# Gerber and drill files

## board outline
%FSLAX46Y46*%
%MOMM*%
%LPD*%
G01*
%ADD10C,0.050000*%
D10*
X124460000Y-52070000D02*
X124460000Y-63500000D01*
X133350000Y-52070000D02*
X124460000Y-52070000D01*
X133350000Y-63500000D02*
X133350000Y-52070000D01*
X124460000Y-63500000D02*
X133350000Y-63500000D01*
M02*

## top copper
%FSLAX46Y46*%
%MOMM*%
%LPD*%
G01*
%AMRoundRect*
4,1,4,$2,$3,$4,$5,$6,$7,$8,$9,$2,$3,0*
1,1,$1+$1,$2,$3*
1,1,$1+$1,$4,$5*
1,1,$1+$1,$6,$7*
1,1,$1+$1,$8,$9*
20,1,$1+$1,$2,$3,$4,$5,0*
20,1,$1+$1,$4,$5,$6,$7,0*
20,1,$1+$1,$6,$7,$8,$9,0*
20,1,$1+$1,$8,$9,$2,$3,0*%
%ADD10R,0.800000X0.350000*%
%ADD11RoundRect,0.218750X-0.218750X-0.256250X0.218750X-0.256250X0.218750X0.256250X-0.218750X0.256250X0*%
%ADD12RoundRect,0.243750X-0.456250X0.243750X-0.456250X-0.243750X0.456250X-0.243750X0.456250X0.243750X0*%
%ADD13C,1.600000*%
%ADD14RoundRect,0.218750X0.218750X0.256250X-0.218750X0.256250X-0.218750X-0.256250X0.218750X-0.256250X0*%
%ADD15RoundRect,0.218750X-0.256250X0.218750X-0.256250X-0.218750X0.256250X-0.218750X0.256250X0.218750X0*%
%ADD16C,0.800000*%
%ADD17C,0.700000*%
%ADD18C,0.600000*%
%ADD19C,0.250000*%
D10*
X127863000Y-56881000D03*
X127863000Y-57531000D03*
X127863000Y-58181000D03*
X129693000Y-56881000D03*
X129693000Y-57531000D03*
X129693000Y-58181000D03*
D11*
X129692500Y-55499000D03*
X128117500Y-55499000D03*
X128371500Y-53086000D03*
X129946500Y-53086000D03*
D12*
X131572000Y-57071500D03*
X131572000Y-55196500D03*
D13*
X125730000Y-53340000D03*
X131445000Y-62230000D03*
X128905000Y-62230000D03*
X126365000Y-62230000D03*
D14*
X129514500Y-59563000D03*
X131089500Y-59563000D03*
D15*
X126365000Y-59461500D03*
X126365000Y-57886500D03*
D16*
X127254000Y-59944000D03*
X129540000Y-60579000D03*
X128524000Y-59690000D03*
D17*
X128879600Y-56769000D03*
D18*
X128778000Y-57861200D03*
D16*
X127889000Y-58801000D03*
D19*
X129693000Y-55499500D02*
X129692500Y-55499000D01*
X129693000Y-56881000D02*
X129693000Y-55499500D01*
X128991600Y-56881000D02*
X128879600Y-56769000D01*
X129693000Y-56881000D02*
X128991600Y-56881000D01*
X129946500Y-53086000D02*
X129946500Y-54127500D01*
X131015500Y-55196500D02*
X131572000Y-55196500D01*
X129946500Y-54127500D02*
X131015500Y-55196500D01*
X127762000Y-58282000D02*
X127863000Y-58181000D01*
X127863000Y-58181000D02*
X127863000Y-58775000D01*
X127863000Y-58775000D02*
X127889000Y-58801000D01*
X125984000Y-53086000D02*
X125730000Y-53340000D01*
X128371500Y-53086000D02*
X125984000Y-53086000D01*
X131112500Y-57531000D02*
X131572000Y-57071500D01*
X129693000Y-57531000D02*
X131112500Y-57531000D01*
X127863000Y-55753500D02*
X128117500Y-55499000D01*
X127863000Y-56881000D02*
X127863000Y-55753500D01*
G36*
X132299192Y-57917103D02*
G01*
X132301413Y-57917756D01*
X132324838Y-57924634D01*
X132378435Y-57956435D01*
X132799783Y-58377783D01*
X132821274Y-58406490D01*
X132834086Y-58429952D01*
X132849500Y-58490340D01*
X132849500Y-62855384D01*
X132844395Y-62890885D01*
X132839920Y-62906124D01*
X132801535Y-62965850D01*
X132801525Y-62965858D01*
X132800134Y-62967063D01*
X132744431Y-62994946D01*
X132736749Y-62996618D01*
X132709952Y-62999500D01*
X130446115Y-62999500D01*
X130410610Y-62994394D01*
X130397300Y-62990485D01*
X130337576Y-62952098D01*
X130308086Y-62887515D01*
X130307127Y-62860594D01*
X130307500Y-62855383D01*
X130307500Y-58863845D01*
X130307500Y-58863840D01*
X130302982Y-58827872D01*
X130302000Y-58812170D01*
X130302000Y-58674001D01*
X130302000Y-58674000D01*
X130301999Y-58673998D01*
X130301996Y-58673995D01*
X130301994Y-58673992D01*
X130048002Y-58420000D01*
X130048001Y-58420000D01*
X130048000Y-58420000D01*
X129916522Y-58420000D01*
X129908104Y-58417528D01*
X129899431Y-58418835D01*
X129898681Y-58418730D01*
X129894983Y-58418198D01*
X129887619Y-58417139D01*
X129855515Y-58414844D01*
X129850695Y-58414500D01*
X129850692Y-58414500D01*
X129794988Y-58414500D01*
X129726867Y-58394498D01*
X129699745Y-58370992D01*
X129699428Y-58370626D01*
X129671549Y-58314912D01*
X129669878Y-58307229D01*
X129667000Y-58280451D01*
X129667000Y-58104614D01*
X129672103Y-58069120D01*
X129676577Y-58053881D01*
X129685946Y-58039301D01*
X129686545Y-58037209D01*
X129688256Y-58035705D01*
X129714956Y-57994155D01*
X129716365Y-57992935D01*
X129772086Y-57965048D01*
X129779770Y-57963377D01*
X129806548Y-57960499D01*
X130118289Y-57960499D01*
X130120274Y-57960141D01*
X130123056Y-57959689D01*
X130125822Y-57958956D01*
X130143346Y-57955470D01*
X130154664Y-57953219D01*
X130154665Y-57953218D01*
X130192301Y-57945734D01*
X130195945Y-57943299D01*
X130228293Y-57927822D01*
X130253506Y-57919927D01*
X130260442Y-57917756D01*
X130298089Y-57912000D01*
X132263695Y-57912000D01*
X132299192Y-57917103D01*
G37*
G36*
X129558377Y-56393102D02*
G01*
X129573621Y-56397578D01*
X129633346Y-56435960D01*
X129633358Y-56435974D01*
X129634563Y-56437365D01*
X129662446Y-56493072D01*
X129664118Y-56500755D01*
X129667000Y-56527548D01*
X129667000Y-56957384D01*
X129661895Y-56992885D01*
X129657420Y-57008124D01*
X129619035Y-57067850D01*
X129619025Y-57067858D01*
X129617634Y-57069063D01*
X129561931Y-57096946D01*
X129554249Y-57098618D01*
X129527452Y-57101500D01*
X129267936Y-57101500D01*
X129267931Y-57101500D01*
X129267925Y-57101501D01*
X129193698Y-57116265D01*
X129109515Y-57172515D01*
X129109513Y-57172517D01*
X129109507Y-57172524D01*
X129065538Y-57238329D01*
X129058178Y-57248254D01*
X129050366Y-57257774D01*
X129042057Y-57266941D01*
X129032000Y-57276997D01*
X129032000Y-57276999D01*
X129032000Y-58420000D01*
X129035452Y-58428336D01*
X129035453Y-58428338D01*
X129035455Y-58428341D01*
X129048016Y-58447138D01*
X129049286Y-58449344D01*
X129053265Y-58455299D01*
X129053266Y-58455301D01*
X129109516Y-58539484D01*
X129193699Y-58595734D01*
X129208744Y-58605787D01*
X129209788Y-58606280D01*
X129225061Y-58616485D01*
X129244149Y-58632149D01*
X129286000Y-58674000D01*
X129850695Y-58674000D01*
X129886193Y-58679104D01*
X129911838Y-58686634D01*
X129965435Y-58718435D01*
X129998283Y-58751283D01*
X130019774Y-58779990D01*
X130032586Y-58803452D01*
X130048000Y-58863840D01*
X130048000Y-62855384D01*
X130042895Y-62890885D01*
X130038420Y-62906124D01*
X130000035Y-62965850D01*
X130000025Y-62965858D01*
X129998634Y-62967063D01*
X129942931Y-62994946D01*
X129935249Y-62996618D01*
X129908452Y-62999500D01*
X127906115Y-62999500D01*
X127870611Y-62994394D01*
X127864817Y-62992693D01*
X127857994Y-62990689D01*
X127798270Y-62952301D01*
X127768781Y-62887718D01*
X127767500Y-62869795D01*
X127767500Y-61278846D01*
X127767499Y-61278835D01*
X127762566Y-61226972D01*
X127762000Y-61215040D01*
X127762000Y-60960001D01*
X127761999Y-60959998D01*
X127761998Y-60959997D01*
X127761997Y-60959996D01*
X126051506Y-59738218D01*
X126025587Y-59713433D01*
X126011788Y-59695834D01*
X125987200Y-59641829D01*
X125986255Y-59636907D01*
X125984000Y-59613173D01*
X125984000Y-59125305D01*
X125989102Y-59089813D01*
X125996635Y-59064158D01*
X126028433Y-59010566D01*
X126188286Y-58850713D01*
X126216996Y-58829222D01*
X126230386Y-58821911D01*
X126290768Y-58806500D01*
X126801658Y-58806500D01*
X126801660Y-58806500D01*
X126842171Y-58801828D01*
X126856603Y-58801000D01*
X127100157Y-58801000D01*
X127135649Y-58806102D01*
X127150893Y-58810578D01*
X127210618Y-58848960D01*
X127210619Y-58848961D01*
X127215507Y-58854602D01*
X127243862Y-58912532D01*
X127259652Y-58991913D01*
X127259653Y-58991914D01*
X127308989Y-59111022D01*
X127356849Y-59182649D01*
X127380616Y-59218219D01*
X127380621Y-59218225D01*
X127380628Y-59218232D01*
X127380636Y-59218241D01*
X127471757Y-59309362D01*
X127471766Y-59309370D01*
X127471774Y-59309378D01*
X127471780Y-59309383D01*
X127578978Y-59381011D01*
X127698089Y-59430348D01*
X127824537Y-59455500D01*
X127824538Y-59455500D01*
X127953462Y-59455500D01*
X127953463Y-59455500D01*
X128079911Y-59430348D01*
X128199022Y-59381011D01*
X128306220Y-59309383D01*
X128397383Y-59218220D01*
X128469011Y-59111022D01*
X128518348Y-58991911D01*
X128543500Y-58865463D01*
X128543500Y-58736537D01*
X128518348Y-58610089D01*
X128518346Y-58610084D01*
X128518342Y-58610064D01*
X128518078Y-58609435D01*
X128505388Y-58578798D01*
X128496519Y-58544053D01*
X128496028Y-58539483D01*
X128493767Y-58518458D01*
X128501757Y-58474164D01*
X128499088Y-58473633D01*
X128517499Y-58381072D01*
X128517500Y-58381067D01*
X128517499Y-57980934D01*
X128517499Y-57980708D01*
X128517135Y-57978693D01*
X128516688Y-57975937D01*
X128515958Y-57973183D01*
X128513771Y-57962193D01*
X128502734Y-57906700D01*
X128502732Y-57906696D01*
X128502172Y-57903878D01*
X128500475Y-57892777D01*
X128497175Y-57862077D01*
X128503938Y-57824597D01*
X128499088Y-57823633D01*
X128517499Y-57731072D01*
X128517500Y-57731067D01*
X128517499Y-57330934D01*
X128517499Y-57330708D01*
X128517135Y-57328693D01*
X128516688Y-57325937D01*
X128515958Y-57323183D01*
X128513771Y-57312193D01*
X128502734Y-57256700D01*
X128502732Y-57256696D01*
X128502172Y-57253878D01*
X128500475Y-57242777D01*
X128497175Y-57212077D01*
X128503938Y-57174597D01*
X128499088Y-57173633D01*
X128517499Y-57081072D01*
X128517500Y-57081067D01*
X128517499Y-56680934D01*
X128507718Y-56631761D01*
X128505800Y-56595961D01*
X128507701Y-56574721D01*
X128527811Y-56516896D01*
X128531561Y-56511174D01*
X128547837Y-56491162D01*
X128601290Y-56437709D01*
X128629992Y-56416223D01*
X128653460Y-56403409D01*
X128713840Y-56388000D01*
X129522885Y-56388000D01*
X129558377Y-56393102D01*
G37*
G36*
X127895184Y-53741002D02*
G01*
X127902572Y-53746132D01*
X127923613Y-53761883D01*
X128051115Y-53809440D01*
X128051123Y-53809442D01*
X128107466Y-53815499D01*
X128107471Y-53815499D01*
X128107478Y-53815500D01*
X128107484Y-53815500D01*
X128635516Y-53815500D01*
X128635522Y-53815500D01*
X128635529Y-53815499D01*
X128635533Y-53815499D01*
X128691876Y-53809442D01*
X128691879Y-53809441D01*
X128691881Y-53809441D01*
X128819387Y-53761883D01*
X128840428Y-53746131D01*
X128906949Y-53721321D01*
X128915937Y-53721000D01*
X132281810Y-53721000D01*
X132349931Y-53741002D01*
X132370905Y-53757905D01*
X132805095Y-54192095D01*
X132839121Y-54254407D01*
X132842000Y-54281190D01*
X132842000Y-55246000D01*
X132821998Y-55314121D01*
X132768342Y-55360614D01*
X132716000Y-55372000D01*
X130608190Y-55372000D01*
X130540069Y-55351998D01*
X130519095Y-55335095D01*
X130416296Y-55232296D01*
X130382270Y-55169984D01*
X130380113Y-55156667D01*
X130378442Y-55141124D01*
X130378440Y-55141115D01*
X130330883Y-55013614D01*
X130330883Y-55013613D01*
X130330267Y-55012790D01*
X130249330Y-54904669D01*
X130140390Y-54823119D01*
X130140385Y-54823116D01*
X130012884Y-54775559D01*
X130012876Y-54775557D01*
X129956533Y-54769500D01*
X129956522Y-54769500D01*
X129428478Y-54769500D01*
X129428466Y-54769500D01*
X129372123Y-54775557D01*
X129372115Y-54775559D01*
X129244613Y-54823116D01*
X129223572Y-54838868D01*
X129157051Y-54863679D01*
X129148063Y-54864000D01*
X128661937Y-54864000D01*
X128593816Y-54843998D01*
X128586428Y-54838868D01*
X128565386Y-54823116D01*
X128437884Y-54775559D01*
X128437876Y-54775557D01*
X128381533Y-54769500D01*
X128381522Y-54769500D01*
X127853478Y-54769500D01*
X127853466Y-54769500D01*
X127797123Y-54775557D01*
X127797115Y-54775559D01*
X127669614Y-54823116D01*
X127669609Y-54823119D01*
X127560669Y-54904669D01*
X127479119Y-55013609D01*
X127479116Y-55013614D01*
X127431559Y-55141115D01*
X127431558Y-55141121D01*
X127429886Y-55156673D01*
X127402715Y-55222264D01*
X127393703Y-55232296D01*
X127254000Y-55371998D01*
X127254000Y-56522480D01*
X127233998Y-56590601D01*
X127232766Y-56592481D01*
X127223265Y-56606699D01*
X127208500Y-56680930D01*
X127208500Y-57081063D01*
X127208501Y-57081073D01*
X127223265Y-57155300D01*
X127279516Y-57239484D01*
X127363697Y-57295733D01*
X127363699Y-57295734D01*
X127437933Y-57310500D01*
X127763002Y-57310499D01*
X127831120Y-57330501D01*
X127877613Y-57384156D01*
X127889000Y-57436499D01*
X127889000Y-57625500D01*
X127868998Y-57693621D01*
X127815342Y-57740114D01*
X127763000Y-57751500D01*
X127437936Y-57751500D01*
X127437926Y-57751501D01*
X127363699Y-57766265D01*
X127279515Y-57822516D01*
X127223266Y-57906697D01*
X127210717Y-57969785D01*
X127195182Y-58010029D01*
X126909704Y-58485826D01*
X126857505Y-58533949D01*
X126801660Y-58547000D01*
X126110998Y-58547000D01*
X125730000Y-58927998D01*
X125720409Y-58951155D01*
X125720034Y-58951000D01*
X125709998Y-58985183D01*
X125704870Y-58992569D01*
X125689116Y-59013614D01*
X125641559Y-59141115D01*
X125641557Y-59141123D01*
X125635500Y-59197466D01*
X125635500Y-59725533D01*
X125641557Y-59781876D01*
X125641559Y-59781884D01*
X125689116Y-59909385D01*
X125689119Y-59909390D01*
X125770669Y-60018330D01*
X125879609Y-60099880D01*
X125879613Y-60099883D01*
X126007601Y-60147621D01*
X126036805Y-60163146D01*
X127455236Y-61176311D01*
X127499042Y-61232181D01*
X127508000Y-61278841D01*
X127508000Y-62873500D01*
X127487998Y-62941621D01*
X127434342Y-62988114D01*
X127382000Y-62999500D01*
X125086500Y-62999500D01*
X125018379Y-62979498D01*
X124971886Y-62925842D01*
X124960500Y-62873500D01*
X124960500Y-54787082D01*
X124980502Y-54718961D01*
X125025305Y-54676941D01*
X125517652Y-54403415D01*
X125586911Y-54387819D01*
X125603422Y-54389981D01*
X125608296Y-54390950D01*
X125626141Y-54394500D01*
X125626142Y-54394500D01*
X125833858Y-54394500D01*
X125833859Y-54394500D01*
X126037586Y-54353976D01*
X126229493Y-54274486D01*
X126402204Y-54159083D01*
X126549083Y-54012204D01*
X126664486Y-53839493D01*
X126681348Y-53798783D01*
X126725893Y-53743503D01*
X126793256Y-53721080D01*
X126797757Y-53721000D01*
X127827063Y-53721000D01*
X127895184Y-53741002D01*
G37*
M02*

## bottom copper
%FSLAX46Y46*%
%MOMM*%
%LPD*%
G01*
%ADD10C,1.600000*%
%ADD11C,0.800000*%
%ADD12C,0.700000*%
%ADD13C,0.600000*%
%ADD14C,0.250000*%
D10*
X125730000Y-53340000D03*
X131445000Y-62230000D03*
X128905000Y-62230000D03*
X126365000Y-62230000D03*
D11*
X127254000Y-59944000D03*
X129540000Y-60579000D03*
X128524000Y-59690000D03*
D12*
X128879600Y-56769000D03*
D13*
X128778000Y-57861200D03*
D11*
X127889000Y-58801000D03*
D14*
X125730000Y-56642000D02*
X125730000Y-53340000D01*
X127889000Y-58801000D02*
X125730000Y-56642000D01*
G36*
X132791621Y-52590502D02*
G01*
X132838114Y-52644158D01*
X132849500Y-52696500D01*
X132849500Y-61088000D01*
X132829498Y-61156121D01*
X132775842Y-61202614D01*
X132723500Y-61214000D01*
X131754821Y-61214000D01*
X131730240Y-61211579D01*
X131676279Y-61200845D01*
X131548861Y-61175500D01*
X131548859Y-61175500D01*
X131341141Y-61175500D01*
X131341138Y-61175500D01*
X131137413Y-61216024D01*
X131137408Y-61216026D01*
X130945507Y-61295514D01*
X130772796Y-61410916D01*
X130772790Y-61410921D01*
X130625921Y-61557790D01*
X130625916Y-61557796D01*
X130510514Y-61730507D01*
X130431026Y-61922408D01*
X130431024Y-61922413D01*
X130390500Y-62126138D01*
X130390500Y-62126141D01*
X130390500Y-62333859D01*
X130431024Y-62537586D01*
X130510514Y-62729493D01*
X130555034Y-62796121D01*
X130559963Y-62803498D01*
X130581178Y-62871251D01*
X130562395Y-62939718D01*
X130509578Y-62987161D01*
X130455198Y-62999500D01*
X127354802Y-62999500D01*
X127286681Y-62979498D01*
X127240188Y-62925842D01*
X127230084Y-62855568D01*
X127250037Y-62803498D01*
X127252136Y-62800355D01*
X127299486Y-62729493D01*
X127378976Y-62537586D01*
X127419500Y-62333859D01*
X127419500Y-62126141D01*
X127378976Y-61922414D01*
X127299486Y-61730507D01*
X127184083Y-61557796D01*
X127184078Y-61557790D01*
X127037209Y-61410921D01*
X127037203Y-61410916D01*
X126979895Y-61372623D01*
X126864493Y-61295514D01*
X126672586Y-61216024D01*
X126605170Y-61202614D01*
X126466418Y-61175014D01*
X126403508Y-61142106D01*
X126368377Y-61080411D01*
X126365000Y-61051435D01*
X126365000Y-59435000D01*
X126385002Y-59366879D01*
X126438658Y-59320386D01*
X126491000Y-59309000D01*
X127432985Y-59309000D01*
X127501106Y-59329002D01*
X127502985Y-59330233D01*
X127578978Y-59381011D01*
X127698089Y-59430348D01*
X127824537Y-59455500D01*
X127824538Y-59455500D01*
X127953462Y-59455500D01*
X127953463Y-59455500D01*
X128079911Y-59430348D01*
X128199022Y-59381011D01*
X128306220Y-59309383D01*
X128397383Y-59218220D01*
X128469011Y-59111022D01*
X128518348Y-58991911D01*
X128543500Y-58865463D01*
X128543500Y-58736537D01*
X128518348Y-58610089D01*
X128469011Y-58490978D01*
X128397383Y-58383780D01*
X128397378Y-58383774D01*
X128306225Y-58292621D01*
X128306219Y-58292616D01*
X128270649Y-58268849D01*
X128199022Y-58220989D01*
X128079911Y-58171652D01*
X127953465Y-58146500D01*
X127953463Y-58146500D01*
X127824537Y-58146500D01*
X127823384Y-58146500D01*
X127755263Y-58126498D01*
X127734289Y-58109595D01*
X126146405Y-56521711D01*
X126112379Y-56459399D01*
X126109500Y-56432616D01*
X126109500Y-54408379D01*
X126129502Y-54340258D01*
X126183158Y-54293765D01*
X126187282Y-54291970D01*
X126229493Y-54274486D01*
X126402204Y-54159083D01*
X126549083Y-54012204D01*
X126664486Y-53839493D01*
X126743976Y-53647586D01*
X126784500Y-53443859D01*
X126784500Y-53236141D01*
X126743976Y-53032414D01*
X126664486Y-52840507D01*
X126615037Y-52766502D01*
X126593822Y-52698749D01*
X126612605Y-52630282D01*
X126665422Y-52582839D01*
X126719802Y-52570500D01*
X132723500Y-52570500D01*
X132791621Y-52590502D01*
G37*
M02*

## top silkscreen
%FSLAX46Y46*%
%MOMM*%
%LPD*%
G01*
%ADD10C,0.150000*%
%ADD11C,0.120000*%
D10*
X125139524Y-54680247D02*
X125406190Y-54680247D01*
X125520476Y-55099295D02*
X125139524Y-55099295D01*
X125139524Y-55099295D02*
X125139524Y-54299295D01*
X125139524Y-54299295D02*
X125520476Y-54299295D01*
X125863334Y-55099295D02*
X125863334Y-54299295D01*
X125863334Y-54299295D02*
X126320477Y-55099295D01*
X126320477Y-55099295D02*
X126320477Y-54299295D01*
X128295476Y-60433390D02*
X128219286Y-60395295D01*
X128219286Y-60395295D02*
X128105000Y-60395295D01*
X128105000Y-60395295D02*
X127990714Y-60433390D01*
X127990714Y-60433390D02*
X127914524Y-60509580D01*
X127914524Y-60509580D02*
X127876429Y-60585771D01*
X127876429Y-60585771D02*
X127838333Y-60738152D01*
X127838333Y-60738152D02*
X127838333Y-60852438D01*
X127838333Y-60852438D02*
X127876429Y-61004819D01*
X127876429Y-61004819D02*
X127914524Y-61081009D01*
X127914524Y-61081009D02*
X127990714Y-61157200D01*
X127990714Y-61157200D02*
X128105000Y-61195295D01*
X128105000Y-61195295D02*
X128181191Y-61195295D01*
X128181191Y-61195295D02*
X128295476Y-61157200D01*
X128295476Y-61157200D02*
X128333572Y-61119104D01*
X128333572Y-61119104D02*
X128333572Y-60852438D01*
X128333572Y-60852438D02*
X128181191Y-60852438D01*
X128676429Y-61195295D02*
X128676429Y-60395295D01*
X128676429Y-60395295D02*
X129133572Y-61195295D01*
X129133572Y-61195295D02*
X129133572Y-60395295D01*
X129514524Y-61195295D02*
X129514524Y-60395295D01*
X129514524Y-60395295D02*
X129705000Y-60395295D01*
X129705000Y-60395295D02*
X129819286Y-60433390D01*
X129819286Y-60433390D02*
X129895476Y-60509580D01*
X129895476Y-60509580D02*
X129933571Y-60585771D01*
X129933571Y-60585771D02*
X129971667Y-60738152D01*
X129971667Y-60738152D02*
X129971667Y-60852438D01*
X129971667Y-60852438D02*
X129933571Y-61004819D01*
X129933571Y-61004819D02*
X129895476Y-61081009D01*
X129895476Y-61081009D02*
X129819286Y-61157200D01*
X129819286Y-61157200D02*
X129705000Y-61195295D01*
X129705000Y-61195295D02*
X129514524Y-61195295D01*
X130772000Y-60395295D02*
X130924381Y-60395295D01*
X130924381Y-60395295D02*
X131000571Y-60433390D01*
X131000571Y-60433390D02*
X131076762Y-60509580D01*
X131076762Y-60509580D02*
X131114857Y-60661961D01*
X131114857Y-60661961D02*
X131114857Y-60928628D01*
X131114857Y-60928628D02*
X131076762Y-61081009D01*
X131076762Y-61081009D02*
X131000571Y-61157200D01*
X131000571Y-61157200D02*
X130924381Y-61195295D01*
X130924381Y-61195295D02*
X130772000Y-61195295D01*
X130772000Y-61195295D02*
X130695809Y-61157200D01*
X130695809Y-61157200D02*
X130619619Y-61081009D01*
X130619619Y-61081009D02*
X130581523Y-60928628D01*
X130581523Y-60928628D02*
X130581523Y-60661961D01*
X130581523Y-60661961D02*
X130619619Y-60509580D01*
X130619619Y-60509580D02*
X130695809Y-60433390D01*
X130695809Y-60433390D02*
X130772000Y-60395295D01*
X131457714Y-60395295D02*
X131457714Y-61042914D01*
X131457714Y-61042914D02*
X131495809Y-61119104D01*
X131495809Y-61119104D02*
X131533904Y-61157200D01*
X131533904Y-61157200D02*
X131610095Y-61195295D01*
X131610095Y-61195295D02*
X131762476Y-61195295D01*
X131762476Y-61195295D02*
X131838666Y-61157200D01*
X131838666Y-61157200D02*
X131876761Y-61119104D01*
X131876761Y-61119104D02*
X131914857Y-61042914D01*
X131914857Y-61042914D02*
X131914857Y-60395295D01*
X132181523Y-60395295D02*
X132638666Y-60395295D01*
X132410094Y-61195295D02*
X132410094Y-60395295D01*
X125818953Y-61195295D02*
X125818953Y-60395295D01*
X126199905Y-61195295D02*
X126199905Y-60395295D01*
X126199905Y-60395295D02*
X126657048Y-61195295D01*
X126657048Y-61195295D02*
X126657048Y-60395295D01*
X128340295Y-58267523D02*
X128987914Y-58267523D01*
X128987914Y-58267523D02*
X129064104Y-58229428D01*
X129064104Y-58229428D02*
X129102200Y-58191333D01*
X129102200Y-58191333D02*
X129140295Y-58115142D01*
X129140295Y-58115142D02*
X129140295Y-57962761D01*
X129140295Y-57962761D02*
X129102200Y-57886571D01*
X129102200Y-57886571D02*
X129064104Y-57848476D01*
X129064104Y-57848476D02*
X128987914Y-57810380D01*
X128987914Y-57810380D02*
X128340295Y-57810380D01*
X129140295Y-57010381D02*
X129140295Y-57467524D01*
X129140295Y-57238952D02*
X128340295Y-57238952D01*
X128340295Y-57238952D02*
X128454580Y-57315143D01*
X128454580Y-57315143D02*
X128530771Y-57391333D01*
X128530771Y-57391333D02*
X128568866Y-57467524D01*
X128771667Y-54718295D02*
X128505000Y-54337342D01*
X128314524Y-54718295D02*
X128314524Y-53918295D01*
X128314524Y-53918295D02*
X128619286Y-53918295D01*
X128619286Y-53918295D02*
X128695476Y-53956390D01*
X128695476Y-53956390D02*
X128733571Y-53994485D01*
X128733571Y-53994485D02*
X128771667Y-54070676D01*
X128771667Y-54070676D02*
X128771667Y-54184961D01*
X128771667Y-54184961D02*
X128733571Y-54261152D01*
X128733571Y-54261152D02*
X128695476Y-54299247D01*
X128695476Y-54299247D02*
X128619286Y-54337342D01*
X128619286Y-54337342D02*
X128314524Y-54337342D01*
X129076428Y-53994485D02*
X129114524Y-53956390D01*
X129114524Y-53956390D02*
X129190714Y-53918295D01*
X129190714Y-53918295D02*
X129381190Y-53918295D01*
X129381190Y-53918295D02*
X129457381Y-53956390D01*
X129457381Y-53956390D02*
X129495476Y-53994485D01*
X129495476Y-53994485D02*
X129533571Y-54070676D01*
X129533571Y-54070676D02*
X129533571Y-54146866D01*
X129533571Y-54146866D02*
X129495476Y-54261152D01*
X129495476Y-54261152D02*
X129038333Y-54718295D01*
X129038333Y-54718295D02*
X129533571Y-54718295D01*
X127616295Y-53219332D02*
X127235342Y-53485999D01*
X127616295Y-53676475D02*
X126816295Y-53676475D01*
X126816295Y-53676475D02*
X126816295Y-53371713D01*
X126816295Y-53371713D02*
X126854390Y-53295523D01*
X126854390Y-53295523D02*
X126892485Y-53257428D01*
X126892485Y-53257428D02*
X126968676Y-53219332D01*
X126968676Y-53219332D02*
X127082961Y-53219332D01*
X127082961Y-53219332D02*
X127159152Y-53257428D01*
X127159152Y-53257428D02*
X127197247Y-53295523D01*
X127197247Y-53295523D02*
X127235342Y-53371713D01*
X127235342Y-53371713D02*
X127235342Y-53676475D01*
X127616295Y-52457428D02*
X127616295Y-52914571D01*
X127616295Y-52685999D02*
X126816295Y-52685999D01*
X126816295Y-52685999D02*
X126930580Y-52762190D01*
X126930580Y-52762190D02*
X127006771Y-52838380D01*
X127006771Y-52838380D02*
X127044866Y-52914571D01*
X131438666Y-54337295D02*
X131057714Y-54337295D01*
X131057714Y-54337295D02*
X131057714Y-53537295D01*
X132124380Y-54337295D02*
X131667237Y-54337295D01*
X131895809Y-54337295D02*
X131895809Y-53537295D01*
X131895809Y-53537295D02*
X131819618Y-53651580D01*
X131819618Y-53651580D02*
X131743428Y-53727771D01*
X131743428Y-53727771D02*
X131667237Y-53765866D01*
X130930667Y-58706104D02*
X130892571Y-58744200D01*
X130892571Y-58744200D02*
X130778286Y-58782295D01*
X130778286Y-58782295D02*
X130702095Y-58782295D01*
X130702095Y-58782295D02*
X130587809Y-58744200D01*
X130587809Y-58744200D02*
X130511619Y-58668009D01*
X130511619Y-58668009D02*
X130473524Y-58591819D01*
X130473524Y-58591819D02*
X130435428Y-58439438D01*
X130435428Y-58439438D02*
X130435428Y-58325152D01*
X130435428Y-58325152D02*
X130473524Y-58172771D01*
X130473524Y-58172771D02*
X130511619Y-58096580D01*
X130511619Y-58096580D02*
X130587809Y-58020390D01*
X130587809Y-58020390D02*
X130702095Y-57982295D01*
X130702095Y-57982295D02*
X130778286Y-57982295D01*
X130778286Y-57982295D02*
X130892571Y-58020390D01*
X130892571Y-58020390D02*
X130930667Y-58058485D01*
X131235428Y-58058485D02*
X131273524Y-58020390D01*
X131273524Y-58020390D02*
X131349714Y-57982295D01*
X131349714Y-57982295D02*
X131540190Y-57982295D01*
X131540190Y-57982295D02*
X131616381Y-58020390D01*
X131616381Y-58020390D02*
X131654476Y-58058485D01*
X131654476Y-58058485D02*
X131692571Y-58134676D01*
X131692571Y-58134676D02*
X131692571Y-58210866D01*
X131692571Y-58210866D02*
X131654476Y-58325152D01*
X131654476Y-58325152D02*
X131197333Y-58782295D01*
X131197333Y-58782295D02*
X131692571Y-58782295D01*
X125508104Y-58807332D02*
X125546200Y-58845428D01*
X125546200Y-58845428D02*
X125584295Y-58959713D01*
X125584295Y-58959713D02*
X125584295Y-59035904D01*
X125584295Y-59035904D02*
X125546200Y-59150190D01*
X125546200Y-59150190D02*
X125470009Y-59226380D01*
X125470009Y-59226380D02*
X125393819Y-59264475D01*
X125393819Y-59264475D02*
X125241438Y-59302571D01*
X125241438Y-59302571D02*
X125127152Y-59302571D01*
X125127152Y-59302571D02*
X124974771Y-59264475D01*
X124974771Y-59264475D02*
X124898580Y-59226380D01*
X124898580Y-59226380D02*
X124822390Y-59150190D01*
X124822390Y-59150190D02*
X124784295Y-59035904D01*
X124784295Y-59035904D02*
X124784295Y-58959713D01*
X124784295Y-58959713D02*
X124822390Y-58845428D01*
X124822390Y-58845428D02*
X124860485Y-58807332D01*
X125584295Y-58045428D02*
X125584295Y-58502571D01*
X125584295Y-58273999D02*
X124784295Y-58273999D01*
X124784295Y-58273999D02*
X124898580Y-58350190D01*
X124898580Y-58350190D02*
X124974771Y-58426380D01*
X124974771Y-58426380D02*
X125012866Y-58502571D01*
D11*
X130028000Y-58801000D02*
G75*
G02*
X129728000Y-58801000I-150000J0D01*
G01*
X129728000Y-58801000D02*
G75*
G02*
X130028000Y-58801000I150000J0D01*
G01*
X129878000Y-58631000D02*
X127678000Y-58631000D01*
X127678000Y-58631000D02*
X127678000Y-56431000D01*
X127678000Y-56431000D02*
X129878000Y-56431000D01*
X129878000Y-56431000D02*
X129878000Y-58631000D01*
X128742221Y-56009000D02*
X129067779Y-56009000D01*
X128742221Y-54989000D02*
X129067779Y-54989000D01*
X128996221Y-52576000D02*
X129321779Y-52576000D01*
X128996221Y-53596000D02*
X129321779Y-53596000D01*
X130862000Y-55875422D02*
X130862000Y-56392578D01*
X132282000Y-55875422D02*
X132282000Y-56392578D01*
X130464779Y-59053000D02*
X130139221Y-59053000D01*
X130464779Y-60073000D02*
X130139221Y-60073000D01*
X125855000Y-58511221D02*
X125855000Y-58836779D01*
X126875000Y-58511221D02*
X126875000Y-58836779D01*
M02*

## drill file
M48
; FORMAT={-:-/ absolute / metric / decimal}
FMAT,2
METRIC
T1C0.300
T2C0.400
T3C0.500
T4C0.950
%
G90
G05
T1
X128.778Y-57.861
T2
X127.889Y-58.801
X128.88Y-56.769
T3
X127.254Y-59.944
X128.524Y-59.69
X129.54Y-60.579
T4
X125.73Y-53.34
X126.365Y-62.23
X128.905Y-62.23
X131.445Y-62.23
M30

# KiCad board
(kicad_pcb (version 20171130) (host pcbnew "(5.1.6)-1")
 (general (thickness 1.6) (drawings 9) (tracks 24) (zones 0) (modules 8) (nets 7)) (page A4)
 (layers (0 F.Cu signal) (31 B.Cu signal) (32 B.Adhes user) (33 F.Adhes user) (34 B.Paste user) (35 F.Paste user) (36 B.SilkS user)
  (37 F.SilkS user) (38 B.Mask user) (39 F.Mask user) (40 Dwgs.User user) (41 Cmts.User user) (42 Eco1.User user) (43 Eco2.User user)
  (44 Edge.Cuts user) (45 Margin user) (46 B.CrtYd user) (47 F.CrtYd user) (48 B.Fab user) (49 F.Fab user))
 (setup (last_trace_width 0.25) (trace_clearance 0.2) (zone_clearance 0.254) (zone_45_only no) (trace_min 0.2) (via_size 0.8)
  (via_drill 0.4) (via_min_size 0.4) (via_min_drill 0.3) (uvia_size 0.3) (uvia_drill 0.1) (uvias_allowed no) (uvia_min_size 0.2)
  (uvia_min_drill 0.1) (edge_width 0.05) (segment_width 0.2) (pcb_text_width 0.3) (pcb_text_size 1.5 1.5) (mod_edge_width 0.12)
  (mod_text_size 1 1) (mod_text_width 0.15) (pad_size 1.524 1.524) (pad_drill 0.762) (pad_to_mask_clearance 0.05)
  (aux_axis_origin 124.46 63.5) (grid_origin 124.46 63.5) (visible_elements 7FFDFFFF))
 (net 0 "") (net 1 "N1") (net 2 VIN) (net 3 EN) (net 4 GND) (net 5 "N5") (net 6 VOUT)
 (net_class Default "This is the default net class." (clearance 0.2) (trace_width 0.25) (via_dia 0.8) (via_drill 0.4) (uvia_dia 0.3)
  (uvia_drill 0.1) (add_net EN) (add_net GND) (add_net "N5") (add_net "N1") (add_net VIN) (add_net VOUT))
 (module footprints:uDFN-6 (layer F.Cu) (at 128.778 57.531 180)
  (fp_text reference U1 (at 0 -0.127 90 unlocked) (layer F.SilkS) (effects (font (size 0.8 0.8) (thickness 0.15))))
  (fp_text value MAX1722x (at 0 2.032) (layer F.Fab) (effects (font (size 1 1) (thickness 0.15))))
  (fp_circle (center -1.1 -1.27) (end -0.95 -1.27) (layer F.SilkS) (width 0.12))
  (fp_line (start -1.1 -1.1) (end 1.1 -1.1) (layer F.SilkS) (width 0.12))
  (fp_line (start 1.1 -1.1) (end 1.1 1.1) (layer F.SilkS) (width 0.12))
  (fp_line (start 1.1 1.1) (end -1.1 1.1) (layer F.SilkS) (width 0.12))
  (fp_line (start -1.1 1.1) (end -1.1 -1.1) (layer F.SilkS) (width 0.12))
  (pad 4 smd rect (at 0.915 0.65 180) (size 0.8 0.35) (layers F.Cu F.Paste F.Mask) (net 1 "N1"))
  (pad 5 smd rect (at 0.915 0 180) (size 0.8 0.35) (layers F.Cu F.Paste F.Mask) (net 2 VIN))
  (pad 6 smd rect (at 0.915 -0.65 180) (size 0.8 0.35) (layers F.Cu F.Paste F.Mask) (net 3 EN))
  (pad 3 smd rect (at -0.915 0.65 180) (size 0.8 0.35) (layers F.Cu F.Paste F.Mask) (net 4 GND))
  (pad 2 smd rect (at -0.915 0 180) (size 0.8 0.35) (layers F.Cu F.Paste F.Mask) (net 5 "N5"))
  (pad 1 smd rect (at -0.915 -0.65 180) (size 0.8 0.35) (layers F.Cu F.Paste F.Mask) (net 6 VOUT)))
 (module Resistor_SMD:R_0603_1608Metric (layer F.Cu) (at 128.905 55.499)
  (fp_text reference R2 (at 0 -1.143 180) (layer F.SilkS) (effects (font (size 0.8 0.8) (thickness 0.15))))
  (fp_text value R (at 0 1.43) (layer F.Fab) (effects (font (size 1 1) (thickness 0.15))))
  (fp_line (start -0.162779 0.51) (end 0.162779 0.51) (layer F.SilkS) (width 0.12))
  (fp_line (start -0.162779 -0.51) (end 0.162779 -0.51) (layer F.SilkS) (width 0.12))
  (pad 2 smd roundrect (at 0.7875 0) (size 0.875 0.95) (layers F.Cu F.Paste F.Mask) (roundrect_rratio 0.25) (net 4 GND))
  (pad 1 smd roundrect (at -0.7875 0) (size 0.875 0.95) (layers F.Cu F.Paste F.Mask) (roundrect_rratio 0.25) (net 1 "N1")))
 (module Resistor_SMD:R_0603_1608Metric (layer F.Cu) (at 129.159 53.086)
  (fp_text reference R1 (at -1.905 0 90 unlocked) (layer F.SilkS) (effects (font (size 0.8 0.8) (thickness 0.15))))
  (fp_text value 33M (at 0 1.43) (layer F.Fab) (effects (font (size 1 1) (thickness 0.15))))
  (fp_line (start -0.162779 -0.51) (end 0.162779 -0.51) (layer F.SilkS) (width 0.12))
  (fp_line (start -0.162779 0.51) (end 0.162779 0.51) (layer F.SilkS) (width 0.12))
  (pad 1 smd roundrect (at -0.7875 0) (size 0.875 0.95) (layers F.Cu F.Paste F.Mask) (roundrect_rratio 0.25) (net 3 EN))
  (pad 2 smd roundrect (at 0.7875 0) (size 0.875 0.95) (layers F.Cu F.Paste F.Mask) (roundrect_rratio 0.25) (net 2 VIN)))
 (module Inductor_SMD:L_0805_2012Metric (layer F.Cu) (at 131.572 56.134 270)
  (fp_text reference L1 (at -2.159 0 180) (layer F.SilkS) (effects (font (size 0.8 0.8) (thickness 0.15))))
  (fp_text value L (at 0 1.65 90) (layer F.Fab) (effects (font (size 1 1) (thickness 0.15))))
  (fp_line (start -0.258578 0.71) (end 0.258578 0.71) (layer F.SilkS) (width 0.12))
  (fp_line (start -0.258578 -0.71) (end 0.258578 -0.71) (layer F.SilkS) (width 0.12))
  (pad 2 smd roundrect (at 0.9375 0 270) (size 0.975 1.4) (layers F.Cu F.Paste F.Mask) (roundrect_rratio 0.25) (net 5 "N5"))
  (pad 1 smd roundrect (at -0.9375 0 270) (size 0.975 1.4) (layers F.Cu F.Paste F.Mask) (roundrect_rratio 0.25) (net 2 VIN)))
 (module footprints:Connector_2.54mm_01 (layer F.Cu) (at 125.73 53.34)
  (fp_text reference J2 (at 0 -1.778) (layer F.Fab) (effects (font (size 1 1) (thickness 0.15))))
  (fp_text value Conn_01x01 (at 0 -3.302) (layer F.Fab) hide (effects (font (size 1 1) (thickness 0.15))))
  (pad 1 thru_hole circle (at 0 0) (size 1.6 1.6) (drill 0.95) (layers *.Cu *.Mask) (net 3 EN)))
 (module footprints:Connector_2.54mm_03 (layer F.Cu) (at 126.365 62.23 90)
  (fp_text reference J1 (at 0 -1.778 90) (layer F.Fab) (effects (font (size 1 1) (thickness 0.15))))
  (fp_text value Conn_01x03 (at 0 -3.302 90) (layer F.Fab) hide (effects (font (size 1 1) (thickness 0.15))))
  (pad 3 thru_hole circle (at 0 5.08 90) (size 1.6 1.6) (drill 0.95) (layers *.Cu *.Mask) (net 6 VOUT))
  (pad 2 thru_hole circle (at 0 2.54 90) (size 1.6 1.6) (drill 0.95) (layers *.Cu *.Mask) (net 4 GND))
  (pad 1 thru_hole circle (at 0 0 90) (size 1.6 1.6) (drill 0.95) (layers *.Cu *.Mask) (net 2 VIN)))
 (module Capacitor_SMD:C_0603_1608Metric (layer F.Cu) (at 130.302 59.563 180)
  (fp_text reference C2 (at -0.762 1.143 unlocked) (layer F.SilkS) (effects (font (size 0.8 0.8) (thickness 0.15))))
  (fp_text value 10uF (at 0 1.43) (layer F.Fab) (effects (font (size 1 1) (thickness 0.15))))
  (fp_line (start -0.162779 0.51) (end 0.162779 0.51) (layer F.SilkS) (width 0.12))
  (fp_line (start -0.162779 -0.51) (end 0.162779 -0.51) (layer F.SilkS) (width 0.12))
  (pad 2 smd roundrect (at 0.7875 0 180) (size 0.875 0.95) (layers F.Cu F.Paste F.Mask) (roundrect_rratio 0.25) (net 4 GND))
  (pad 1 smd roundrect (at -0.7875 0 180) (size 0.875 0.95) (layers F.Cu F.Paste F.Mask) (roundrect_rratio 0.25) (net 6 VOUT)))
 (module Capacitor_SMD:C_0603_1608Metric (layer F.Cu) (at 126.365 58.674 270)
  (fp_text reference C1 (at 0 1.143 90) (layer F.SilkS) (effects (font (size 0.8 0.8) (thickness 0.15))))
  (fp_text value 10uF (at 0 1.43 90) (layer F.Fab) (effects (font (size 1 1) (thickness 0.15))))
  (fp_line (start -0.162779 0.51) (end 0.162779 0.51) (layer F.SilkS) (width 0.12))
  (fp_line (start -0.162779 -0.51) (end 0.162779 -0.51) (layer F.SilkS) (width 0.12))
  (pad 2 smd roundrect (at 0.7875 0 270) (size 0.875 0.95) (layers F.Cu F.Paste F.Mask) (roundrect_rratio 0.25) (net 4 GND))
  (pad 1 smd roundrect (at -0.7875 0 270) (size 0.875 0.95) (layers F.Cu F.Paste F.Mask) (roundrect_rratio 0.25) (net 2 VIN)))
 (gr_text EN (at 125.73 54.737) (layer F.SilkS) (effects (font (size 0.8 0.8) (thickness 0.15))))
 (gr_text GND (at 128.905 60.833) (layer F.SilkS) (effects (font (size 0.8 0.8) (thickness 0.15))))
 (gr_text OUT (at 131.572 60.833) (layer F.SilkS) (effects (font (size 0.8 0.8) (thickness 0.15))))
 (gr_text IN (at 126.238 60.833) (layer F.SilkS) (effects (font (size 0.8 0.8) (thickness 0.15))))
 (gr_line (start 124.46 52.07) (end 124.46 63.5) (layer Edge.Cuts) (width 0.05))
 (gr_line (start 133.35 52.07) (end 124.46 52.07) (layer Edge.Cuts) (width 0.05))
 (gr_line (start 133.35 63.5) (end 133.35 52.07) (layer Edge.Cuts) (width 0.05))
 (gr_line (start 124.46 63.5) (end 133.35 63.5) (layer Edge.Cuts) (width 0.05))
 (segment (start 129.693 55.4995) (end 129.6925 55.499) (width 0.25) (layer F.Cu) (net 4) (status 30))
 (segment (start 129.693 56.881) (end 129.693 55.4995) (width 0.25) (layer F.Cu) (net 4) (status 30))
 (via (at 127.254 59.944) (size 0.8) (drill 0.5) (layers F.Cu B.Cu) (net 4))
 (via (at 129.54 60.579) (size 0.8) (drill 0.5) (layers F.Cu B.Cu) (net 4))
 (via (at 128.524 59.69) (size 0.8) (drill 0.5) (layers F.Cu B.Cu) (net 4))
 (via (at 128.8796 56.769) (size 0.7) (drill 0.4) (layers F.Cu B.Cu) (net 4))
 (segment (start 128.9916 56.881) (end 128.8796 56.769) (width 0.25) (layer F.Cu) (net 4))
 (segment (start 129.693 56.881) (end 128.9916 56.881) (width 0.25) (layer F.Cu) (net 4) (status 10))
 (via (at 128.778 57.8612) (size 0.6) (drill 0.3) (layers F.Cu B.Cu) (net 4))
 (segment (start 129.9465 53.086) (end 129.9465 54.1275) (width 0.25) (layer F.Cu) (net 2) (status 10))
 (segment (start 131.0155 55.1965) (end 131.572 55.1965) (width 0.25) (layer F.Cu) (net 2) (status 30))
 (segment (start 129.9465 54.1275) (end 131.0155 55.1965) (width 0.25) (layer F.Cu) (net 2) (status 20))
 (segment (start 127.762 58.282) (end 127.863 58.181) (width 0.25) (layer F.Cu) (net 3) (status 30))
 (via (at 127.889 58.801) (size 0.8) (drill 0.4) (layers F.Cu B.Cu) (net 3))
 (segment (start 127.863 58.181) (end 127.863 58.775) (width 0.25) (layer F.Cu) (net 3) (status 10))
 (segment (start 127.863 58.775) (end 127.889 58.801) (width 0.25) (layer F.Cu) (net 3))
 (segment (start 125.73 56.642) (end 125.73 53.34) (width 0.25) (layer B.Cu) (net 3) (status 20))
 (segment (start 127.889 58.801) (end 125.73 56.642) (width 0.25) (layer B.Cu) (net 3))
 (segment (start 125.984 53.086) (end 125.73 53.34) (width 0.25) (layer F.Cu) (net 3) (status 30))
 (segment (start 128.3715 53.086) (end 125.984 53.086) (width 0.25) (layer F.Cu) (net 3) (status 30))
 (segment (start 131.1125 57.531) (end 131.572 57.0715) (width 0.25) (layer F.Cu) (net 5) (status 30))
 (segment (start 129.693 57.531) (end 131.1125 57.531) (width 0.25) (layer F.Cu) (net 5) (status 30))
 (segment (start 127.863 55.7535) (end 128.1175 55.499) (width 0.25) (layer F.Cu) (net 1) (status 30))
 (segment (start 127.863 56.881) (end 127.863 55.7535) (width 0.25) (layer F.Cu) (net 1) (status 30))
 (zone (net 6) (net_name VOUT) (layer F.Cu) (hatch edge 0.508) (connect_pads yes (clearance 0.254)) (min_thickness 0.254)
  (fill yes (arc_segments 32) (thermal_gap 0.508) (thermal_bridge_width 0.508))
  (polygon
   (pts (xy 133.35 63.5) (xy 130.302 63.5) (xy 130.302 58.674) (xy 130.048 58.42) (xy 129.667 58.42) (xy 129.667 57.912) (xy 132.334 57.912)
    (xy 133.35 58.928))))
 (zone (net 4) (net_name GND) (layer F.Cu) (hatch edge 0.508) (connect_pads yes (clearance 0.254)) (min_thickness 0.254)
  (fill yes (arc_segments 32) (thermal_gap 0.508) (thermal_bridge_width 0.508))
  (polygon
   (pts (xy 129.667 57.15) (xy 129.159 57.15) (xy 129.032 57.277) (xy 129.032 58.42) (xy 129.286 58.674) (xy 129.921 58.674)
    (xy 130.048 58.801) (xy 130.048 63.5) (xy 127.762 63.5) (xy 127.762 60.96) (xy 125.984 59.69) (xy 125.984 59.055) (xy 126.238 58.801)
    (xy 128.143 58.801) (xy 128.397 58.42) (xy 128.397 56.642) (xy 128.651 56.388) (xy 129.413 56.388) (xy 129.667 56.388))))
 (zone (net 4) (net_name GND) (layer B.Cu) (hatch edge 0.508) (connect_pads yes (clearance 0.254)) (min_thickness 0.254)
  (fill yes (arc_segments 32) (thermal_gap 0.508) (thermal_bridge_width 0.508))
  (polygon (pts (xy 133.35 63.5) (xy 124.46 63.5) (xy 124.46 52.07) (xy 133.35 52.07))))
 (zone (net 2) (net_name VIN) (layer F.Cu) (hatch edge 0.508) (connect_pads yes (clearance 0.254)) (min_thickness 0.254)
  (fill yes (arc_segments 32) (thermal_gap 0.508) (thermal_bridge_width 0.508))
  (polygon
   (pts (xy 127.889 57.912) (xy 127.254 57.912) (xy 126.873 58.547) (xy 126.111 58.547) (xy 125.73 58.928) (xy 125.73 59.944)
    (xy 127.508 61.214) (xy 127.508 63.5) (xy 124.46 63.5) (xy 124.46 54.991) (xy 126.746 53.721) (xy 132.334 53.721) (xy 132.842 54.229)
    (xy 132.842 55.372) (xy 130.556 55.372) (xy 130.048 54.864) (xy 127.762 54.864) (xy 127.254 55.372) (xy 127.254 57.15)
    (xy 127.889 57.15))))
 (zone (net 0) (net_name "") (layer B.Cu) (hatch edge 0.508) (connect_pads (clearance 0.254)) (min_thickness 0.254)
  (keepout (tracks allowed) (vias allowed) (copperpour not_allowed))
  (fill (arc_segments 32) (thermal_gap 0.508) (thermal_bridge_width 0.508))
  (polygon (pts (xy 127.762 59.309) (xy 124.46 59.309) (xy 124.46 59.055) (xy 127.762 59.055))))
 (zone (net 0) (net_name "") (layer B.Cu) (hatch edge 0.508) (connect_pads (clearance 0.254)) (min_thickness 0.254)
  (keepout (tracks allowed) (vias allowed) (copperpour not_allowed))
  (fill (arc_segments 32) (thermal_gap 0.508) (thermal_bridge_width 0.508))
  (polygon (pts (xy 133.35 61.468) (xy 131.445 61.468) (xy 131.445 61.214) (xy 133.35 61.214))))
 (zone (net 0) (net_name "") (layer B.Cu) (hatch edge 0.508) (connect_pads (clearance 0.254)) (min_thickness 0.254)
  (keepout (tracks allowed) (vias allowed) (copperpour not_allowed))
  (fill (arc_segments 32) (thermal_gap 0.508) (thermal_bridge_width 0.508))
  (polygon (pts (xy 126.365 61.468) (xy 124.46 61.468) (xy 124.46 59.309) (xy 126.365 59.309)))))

